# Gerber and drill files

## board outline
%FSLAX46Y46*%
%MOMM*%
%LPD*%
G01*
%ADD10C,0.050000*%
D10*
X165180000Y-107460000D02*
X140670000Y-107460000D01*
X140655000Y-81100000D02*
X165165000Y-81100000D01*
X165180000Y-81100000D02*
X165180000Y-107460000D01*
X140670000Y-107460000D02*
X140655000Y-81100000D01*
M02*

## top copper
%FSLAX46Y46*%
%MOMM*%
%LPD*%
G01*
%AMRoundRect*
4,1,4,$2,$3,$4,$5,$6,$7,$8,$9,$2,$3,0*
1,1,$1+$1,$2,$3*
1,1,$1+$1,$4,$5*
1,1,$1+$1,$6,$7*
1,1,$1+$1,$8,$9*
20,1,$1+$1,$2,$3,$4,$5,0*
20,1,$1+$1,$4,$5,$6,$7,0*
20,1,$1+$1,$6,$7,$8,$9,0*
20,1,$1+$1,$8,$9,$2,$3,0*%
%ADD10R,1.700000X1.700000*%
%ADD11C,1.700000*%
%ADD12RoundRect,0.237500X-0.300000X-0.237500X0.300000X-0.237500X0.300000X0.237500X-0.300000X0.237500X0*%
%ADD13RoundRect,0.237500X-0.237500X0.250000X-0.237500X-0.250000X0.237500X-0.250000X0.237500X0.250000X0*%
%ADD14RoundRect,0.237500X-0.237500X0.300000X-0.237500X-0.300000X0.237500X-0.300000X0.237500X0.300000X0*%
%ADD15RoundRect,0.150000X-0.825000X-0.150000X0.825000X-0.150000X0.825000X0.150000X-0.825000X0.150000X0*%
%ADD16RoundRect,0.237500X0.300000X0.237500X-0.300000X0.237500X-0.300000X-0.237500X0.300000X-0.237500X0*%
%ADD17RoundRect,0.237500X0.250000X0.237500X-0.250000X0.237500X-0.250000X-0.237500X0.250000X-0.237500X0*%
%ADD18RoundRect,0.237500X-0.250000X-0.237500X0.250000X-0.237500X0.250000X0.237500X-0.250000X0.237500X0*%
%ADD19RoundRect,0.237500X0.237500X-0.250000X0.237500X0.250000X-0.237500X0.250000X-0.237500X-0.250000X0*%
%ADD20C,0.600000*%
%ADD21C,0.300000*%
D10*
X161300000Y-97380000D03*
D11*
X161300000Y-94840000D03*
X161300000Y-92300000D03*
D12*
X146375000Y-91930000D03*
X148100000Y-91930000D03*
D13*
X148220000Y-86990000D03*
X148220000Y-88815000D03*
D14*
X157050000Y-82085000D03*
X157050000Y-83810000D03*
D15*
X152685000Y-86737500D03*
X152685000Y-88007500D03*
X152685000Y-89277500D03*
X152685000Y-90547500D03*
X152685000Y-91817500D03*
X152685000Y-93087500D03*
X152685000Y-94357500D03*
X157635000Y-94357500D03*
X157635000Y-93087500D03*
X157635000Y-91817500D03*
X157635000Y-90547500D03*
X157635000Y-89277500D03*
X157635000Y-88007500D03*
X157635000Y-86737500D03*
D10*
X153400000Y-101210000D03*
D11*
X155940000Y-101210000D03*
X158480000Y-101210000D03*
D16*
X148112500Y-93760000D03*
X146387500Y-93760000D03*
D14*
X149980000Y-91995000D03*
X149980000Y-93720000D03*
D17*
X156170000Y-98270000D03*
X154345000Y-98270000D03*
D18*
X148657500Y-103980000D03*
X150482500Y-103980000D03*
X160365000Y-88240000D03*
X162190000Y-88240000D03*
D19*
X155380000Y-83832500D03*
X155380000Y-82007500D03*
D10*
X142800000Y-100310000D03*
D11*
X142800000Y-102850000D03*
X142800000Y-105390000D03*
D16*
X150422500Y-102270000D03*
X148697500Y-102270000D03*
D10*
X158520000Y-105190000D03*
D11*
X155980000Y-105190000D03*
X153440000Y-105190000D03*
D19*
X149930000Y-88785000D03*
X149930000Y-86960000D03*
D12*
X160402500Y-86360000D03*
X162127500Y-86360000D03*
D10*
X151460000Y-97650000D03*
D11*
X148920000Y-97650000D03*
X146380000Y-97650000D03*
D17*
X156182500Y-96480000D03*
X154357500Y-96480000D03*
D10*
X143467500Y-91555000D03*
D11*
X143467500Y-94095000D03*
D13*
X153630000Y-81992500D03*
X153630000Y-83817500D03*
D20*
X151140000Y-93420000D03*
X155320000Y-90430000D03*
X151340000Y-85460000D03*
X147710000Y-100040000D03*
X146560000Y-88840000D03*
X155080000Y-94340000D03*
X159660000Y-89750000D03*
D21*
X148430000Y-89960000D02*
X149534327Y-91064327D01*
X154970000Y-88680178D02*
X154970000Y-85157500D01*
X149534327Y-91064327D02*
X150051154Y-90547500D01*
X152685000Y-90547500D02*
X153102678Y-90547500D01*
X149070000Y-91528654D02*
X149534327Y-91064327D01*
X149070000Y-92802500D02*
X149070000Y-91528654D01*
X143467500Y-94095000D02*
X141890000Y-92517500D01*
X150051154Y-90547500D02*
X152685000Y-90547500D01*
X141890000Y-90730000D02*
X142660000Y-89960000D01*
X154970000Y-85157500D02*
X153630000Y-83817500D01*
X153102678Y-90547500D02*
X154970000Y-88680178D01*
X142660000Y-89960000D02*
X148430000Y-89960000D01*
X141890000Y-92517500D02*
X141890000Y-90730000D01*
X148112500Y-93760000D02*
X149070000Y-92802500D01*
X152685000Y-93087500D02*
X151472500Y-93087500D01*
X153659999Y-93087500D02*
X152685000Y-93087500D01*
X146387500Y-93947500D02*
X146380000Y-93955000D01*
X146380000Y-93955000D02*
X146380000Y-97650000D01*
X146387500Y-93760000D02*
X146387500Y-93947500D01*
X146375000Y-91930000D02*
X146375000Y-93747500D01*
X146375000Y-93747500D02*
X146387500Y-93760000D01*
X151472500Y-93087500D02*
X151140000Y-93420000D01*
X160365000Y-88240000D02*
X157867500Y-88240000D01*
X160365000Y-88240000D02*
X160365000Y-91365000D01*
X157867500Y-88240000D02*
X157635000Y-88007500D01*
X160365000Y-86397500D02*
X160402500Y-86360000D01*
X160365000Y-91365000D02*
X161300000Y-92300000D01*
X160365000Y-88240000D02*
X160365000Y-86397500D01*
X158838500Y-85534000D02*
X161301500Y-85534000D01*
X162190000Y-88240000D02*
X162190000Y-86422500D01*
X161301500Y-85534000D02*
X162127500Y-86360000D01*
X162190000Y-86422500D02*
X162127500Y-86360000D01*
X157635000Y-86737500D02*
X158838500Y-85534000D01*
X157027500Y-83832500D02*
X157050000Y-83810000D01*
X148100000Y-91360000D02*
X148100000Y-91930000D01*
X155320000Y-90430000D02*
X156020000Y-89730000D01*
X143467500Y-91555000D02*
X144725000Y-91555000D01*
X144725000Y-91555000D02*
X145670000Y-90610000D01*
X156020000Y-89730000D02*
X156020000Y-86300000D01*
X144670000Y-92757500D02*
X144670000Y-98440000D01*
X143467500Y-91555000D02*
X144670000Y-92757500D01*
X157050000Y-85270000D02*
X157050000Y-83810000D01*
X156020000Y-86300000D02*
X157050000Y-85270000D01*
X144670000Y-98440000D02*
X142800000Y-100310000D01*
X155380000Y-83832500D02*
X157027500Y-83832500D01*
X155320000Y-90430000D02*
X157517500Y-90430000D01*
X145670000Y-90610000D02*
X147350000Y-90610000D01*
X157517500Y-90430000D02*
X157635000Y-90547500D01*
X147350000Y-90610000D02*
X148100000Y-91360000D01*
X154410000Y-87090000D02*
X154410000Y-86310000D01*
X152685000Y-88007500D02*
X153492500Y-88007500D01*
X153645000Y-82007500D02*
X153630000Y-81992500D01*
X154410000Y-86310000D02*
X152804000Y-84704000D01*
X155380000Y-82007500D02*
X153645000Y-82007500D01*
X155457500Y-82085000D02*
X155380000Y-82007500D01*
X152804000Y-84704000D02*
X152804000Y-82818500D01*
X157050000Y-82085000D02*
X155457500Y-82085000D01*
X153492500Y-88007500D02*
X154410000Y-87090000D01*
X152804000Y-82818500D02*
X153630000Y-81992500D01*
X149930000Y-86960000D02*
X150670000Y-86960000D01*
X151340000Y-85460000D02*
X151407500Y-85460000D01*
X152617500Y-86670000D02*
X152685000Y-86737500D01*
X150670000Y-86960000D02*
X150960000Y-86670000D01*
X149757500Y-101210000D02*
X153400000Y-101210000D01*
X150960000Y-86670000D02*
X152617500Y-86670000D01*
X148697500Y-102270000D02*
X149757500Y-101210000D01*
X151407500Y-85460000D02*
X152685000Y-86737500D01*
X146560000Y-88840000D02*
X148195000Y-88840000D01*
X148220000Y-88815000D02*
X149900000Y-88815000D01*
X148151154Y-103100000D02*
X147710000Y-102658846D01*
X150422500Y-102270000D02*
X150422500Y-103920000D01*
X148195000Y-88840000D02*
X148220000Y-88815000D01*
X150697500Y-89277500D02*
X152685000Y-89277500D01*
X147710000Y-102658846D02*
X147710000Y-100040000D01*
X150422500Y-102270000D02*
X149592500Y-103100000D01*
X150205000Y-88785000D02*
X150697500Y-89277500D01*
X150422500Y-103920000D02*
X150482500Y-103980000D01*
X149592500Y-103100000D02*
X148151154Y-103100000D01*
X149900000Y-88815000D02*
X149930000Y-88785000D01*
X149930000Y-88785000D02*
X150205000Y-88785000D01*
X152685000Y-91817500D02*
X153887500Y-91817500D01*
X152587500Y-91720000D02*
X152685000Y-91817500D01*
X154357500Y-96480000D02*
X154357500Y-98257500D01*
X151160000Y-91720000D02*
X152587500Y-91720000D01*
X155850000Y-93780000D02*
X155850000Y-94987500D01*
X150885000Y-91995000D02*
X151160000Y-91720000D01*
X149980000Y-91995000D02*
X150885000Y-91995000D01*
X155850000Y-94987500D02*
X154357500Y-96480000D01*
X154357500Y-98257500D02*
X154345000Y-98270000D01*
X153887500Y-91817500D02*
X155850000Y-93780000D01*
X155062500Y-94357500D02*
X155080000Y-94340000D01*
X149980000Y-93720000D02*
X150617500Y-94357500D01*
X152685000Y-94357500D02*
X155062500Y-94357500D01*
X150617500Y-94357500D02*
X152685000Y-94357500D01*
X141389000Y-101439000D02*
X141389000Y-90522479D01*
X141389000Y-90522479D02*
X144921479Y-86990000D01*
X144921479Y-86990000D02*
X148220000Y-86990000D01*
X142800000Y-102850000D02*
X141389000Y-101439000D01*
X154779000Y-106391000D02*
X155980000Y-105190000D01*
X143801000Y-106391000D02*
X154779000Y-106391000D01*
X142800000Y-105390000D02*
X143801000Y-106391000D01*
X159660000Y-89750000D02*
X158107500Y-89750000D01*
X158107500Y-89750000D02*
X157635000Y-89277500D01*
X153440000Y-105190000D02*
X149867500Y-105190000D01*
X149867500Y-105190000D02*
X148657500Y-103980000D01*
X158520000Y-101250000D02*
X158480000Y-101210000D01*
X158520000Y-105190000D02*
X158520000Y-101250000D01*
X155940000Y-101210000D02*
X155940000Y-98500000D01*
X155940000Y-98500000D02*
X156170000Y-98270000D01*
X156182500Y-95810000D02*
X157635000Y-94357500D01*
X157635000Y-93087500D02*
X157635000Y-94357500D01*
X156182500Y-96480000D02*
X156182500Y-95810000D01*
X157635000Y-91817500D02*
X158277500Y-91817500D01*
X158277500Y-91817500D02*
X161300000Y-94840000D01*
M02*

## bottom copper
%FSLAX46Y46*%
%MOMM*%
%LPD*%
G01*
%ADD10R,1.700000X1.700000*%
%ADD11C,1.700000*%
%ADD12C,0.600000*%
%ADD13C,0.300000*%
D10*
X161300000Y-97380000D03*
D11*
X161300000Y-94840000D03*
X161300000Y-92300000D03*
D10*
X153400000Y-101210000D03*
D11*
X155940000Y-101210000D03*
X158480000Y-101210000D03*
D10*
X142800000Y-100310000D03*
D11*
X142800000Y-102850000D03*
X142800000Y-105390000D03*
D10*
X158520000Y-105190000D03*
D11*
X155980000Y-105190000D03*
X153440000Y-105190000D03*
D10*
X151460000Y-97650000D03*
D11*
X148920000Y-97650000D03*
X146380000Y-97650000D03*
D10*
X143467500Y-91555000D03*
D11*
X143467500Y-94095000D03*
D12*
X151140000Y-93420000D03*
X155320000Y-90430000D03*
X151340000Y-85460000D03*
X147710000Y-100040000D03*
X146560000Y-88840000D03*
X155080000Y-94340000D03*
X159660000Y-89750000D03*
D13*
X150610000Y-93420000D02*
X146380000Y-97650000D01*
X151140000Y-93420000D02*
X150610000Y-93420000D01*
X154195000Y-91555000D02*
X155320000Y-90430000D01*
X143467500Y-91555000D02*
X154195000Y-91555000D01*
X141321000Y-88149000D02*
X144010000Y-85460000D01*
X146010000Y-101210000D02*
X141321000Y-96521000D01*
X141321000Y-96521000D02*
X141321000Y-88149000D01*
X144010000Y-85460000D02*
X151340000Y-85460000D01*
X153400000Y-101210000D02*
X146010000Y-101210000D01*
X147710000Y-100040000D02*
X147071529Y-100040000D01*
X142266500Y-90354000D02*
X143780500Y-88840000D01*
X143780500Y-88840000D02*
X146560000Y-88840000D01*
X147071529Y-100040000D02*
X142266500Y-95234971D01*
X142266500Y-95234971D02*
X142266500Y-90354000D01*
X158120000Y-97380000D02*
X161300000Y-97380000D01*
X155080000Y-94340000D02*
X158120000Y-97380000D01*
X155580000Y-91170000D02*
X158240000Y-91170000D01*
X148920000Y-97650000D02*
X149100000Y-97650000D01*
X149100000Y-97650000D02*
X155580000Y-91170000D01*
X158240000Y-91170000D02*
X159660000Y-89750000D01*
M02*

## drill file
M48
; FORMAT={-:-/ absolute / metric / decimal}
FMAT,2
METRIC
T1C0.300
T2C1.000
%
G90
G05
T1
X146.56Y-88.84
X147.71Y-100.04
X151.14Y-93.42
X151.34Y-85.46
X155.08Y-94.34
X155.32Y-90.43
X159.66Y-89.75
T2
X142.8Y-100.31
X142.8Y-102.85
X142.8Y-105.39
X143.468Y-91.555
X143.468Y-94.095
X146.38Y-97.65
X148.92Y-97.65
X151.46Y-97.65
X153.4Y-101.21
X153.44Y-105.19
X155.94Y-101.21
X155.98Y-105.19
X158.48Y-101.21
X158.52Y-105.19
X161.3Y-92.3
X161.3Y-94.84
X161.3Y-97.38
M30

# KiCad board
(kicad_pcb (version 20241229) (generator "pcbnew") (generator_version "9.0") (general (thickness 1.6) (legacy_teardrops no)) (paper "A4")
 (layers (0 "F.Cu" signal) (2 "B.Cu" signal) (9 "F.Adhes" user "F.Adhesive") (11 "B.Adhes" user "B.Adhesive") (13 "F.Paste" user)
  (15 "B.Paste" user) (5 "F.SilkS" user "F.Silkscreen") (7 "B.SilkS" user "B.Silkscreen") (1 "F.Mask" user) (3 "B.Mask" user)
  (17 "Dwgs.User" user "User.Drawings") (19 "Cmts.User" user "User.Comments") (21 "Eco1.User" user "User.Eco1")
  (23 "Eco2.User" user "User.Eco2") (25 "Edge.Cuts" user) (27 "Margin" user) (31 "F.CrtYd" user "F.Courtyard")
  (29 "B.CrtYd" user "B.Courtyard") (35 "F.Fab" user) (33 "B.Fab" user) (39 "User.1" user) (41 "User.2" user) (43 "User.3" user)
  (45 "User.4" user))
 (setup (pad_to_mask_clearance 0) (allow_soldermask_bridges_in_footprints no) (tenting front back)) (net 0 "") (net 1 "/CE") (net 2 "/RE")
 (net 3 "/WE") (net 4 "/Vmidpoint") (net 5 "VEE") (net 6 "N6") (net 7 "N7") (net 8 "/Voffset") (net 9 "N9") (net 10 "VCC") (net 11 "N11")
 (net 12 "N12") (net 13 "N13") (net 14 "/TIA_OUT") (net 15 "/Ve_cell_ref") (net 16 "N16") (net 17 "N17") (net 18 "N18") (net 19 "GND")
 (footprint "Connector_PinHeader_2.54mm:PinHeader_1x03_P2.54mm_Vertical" (layer "F.Cu") (at 161.3 97.38 180)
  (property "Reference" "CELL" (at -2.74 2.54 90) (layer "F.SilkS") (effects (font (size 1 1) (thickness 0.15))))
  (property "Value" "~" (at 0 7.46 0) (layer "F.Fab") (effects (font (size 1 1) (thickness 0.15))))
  (pad "1" thru_hole rect (at 0 0 180) (size 1.7 1.7) (drill 1) (layers "*.Cu" "*.Mask") (remove_unused_layers no) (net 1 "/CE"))
  (pad "2" thru_hole circle (at 0 2.54 180) (size 1.7 1.7) (drill 1) (layers "*.Cu" "*.Mask") (remove_unused_layers no) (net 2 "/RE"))
  (pad "3" thru_hole circle (at 0 5.08 180) (size 1.7 1.7) (drill 1) (layers "*.Cu" "*.Mask") (remove_unused_layers no) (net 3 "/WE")))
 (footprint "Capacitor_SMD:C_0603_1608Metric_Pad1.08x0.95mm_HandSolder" (layer "F.Cu") (at 147.2375 91.93)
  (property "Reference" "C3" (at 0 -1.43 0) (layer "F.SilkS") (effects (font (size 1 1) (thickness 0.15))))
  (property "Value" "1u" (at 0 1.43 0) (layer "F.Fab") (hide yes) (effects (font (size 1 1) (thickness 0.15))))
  (pad "1" smd roundrect (at -0.8625 0) (size 1.075 0.95) (layers "F.Cu" "F.Mask" "F.Paste") (roundrect_rratio 0.25) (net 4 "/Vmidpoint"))
  (pad "2" smd roundrect (at 0.8625 0) (size 1.075 0.95) (layers "F.Cu" "F.Mask" "F.Paste") (roundrect_rratio 0.25) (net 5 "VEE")))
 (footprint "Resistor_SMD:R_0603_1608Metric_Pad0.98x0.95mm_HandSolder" (layer "F.Cu") (at 148.22 87.9025 -90)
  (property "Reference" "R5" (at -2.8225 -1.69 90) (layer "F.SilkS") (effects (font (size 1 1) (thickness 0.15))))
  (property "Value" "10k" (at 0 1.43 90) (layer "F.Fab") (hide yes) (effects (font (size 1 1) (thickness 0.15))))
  (pad "1" smd roundrect (at -0.9125 0 270) (size 0.975 0.95) (layers "F.Cu" "F.Mask" "F.Paste") (roundrect_rratio 0.25) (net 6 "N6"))
  (pad "2" smd roundrect (at 0.9125 0 270) (size 0.975 0.95) (layers "F.Cu" "F.Mask" "F.Paste") (roundrect_rratio 0.25) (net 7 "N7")))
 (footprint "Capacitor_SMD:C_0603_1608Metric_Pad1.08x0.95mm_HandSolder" (layer "F.Cu") (at 157.05 82.9475 -90)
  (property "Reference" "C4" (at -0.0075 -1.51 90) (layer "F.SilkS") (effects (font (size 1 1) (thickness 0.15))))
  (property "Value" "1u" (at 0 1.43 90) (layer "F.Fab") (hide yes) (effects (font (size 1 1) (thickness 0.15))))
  (pad "1" smd roundrect (at -0.8625 0 270) (size 1.075 0.95) (layers "F.Cu" "F.Mask" "F.Paste") (roundrect_rratio 0.25) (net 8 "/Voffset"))
  (pad "2" smd roundrect (at 0.8625 0 270) (size 1.075 0.95) (layers "F.Cu" "F.Mask" "F.Paste") (roundrect_rratio 0.25) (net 5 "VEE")))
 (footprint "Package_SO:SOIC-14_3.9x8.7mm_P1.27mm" (layer "F.Cu") (at 155.16 90.5475)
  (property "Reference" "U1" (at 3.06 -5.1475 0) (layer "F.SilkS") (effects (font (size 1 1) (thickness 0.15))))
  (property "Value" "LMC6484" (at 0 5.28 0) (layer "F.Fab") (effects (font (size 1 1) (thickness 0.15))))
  (pad "1" smd roundrect (at -2.475 -3.81) (size 1.95 0.6) (layers "F.Cu" "F.Mask" "F.Paste") (roundrect_rratio 0.25) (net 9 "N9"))
  (pad "2" smd roundrect (at -2.475 -2.54) (size 1.95 0.6) (layers "F.Cu" "F.Mask" "F.Paste") (roundrect_rratio 0.25) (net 8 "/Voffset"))
  (pad "3" smd roundrect (at -2.475 -1.27) (size 1.95 0.6) (layers "F.Cu" "F.Mask" "F.Paste") (roundrect_rratio 0.25) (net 7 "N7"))
  (pad "4" smd roundrect (at -2.475 0) (size 1.95 0.6) (layers "F.Cu" "F.Mask" "F.Paste") (roundrect_rratio 0.25) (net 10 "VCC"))
  (pad "5" smd roundrect (at -2.475 1.27) (size 1.95 0.6) (layers "F.Cu" "F.Mask" "F.Paste") (roundrect_rratio 0.25) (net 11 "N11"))
  (pad "6" smd roundrect (at -2.475 2.54) (size 1.95 0.6) (layers "F.Cu" "F.Mask" "F.Paste") (roundrect_rratio 0.25) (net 4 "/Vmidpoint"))
  (pad "7" smd roundrect (at -2.475 3.81) (size 1.95 0.6) (layers "F.Cu" "F.Mask" "F.Paste") (roundrect_rratio 0.25) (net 1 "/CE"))
  (pad "8" smd roundrect (at 2.475 3.81) (size 1.95 0.6) (layers "F.Cu" "F.Mask" "F.Paste") (roundrect_rratio 0.25) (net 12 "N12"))
  (pad "9" smd roundrect (at 2.475 2.54) (size 1.95 0.6) (layers "F.Cu" "F.Mask" "F.Paste") (roundrect_rratio 0.25) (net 12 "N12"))
  (pad "10" smd roundrect (at 2.475 1.27) (size 1.95 0.6) (layers "F.Cu" "F.Mask" "F.Paste") (roundrect_rratio 0.25) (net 2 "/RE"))
  (pad "11" smd roundrect (at 2.475 0) (size 1.95 0.6) (layers "F.Cu" "F.Mask" "F.Paste") (roundrect_rratio 0.25) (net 5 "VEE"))
  (pad "12" smd roundrect (at 2.475 -1.27) (size 1.95 0.6) (layers "F.Cu" "F.Mask" "F.Paste") (roundrect_rratio 0.25) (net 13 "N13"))
  (pad "13" smd roundrect (at 2.475 -2.54) (size 1.95 0.6) (layers "F.Cu" "F.Mask" "F.Paste") (roundrect_rratio 0.25) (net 3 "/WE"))
  (pad "14" smd roundrect (at 2.475 -3.81) (size 1.95 0.6) (layers "F.Cu" "F.Mask" "F.Paste") (roundrect_rratio 0.25) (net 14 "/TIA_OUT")))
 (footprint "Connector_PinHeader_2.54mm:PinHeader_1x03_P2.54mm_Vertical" (layer "F.Cu") (at 153.4 101.21 90)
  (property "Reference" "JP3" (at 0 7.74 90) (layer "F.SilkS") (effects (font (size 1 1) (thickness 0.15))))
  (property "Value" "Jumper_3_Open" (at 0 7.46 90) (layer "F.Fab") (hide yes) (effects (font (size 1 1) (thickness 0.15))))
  (pad "1" thru_hole rect (at 0 0 90) (size 1.7 1.7) (drill 1) (layers "*.Cu" "*.Mask") (remove_unused_layers no) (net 9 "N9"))
  (pad "2" thru_hole circle (at 0 2.54 90) (size 1.7 1.7) (drill 1) (layers "*.Cu" "*.Mask") (remove_unused_layers no)
   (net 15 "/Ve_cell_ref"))
  (pad "3" thru_hole circle (at 0 5.08 90) (size 1.7 1.7) (drill 1) (layers "*.Cu" "*.Mask") (remove_unused_layers no) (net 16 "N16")))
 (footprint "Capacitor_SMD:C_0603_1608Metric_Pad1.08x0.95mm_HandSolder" (layer "F.Cu") (at 147.25 93.76 180)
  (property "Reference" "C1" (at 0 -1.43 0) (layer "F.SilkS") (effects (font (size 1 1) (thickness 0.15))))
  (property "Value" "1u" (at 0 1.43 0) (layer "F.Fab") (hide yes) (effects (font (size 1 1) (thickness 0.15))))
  (pad "1" smd roundrect (at -0.8625 0 180) (size 1.075 0.95) (layers "F.Cu" "F.Mask" "F.Paste") (roundrect_rratio 0.25) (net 10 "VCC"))
  (pad "2" smd roundrect (at 0.8625 0 180) (size 1.075 0.95) (layers "F.Cu" "F.Mask" "F.Paste") (roundrect_rratio 0.25) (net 4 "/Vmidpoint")))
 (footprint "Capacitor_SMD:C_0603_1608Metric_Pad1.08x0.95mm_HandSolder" (layer "F.Cu") (at 149.98 92.8575 -90)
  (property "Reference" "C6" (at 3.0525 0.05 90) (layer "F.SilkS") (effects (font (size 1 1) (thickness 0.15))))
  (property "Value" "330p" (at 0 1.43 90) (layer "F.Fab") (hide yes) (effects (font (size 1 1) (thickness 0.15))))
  (pad "1" smd roundrect (at -0.8625 0 270) (size 1.075 0.95) (layers "F.Cu" "F.Mask" "F.Paste") (roundrect_rratio 0.25) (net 11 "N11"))
  (pad "2" smd roundrect (at 0.8625 0 270) (size 1.075 0.95) (layers "F.Cu" "F.Mask" "F.Paste") (roundrect_rratio 0.25) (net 1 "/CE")))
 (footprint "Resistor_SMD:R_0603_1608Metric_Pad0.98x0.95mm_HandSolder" (layer "F.Cu") (at 155.2575 98.27 180)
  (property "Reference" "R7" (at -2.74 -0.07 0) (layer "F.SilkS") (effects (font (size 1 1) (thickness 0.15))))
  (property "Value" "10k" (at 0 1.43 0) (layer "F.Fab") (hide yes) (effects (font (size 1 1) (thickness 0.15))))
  (pad "1" smd roundrect (at -0.9125 0 180) (size 0.975 0.95) (layers "F.Cu" "F.Mask" "F.Paste") (roundrect_rratio 0.25)
   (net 15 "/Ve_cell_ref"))
  (pad "2" smd roundrect (at 0.9125 0 180) (size 0.975 0.95) (layers "F.Cu" "F.Mask" "F.Paste") (roundrect_rratio 0.25) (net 11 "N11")))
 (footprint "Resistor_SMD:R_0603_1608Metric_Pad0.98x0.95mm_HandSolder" (layer "F.Cu") (at 149.57 103.98)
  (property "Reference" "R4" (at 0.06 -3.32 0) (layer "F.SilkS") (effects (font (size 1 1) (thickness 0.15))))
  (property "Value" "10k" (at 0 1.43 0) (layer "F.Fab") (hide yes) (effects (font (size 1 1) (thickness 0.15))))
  (pad "1" smd roundrect (at -0.9125 0) (size 0.975 0.95) (layers "F.Cu" "F.Mask" "F.Paste") (roundrect_rratio 0.25) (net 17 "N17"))
  (pad "2" smd roundrect (at 0.9125 0) (size 0.975 0.95) (layers "F.Cu" "F.Mask" "F.Paste") (roundrect_rratio 0.25) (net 7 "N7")))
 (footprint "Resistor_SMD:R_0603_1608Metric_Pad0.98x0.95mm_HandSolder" (layer "F.Cu") (at 161.2775 88.24)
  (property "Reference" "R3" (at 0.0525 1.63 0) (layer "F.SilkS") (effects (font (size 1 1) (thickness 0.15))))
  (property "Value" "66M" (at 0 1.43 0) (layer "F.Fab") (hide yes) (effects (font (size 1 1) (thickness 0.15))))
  (pad "1" smd roundrect (at -0.9125 0) (size 0.975 0.95) (layers "F.Cu" "F.Mask" "F.Paste") (roundrect_rratio 0.25) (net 3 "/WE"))
  (pad "2" smd roundrect (at 0.9125 0) (size 0.975 0.95) (layers "F.Cu" "F.Mask" "F.Paste") (roundrect_rratio 0.25) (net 14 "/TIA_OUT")))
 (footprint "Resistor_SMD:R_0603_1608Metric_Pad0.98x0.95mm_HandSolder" (layer "F.Cu") (at 155.38 82.92 90)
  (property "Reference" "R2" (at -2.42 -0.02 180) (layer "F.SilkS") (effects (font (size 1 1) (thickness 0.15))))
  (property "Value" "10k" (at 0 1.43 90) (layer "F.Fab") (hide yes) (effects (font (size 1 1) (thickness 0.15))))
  (pad "1" smd roundrect (at -0.9125 0 90) (size 0.975 0.95) (layers "F.Cu" "F.Mask" "F.Paste") (roundrect_rratio 0.25) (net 5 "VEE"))
  (pad "2" smd roundrect (at 0.9125 0 90) (size 0.975 0.95) (layers "F.Cu" "F.Mask" "F.Paste") (roundrect_rratio 0.25) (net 8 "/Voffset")))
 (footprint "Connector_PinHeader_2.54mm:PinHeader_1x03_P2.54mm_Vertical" (layer "F.Cu") (at 142.8 100.31)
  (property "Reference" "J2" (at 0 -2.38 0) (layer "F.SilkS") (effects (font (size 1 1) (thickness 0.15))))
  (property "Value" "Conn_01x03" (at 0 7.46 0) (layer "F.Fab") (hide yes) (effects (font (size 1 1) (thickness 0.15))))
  (pad "1" thru_hole rect (at 0 0) (size 1.7 1.7) (drill 1) (layers "*.Cu" "*.Mask") (remove_unused_layers no) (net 5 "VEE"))
  (pad "2" thru_hole circle (at 0 2.54) (size 1.7 1.7) (drill 1) (layers "*.Cu" "*.Mask") (remove_unused_layers no) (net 6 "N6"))
  (pad "3" thru_hole circle (at 0 5.08) (size 1.7 1.7) (drill 1) (layers "*.Cu" "*.Mask") (remove_unused_layers no) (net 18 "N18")))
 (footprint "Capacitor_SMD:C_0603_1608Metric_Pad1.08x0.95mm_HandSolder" (layer "F.Cu") (at 149.56 102.27 180)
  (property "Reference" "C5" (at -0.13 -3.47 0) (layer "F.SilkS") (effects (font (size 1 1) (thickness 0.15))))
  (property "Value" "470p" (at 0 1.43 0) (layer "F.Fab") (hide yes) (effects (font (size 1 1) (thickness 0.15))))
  (pad "1" smd roundrect (at -0.8625 0 180) (size 1.075 0.95) (layers "F.Cu" "F.Mask" "F.Paste") (roundrect_rratio 0.25) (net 7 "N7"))
  (pad "2" smd roundrect (at 0.8625 0 180) (size 1.075 0.95) (layers "F.Cu" "F.Mask" "F.Paste") (roundrect_rratio 0.25) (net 9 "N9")))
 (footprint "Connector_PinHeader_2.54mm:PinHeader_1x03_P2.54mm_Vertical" (layer "F.Cu") (at 158.52 105.19 -90)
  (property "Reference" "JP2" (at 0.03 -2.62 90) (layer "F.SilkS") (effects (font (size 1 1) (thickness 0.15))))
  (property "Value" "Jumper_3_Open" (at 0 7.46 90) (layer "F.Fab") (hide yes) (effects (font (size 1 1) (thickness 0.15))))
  (pad "1" thru_hole rect (at 0 0 270) (size 1.7 1.7) (drill 1) (layers "*.Cu" "*.Mask") (remove_unused_layers no) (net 16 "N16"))
  (pad "2" thru_hole circle (at 0 2.54 270) (size 1.7 1.7) (drill 1) (layers "*.Cu" "*.Mask") (remove_unused_layers no) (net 18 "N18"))
  (pad "3" thru_hole circle (at 0 5.08 270) (size 1.7 1.7) (drill 1) (layers "*.Cu" "*.Mask") (remove_unused_layers no) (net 17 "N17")))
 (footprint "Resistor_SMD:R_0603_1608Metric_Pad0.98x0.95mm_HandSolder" (layer "F.Cu") (at 149.93 87.8725 90)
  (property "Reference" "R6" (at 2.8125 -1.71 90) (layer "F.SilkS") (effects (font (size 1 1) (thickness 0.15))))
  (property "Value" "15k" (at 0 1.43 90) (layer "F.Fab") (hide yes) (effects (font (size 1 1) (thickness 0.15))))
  (pad "1" smd roundrect (at -0.9125 0 90) (size 0.975 0.95) (layers "F.Cu" "F.Mask" "F.Paste") (roundrect_rratio 0.25) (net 7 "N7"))
  (pad "2" smd roundrect (at 0.9125 0 90) (size 0.975 0.95) (layers "F.Cu" "F.Mask" "F.Paste") (roundrect_rratio 0.25) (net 9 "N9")))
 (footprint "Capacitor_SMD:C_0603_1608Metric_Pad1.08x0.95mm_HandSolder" (layer "F.Cu") (at 161.265 86.36)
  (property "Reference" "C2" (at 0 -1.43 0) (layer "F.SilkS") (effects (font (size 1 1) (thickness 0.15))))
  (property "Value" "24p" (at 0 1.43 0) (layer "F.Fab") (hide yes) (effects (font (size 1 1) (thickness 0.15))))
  (pad "1" smd roundrect (at -0.8625 0) (size 1.075 0.95) (layers "F.Cu" "F.Mask" "F.Paste") (roundrect_rratio 0.25) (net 3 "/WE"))
  (pad "2" smd roundrect (at 0.8625 0) (size 1.075 0.95) (layers "F.Cu" "F.Mask" "F.Paste") (roundrect_rratio 0.25) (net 14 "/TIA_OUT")))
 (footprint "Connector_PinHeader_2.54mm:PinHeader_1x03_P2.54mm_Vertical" (layer "F.Cu") (at 151.46 97.65 -90)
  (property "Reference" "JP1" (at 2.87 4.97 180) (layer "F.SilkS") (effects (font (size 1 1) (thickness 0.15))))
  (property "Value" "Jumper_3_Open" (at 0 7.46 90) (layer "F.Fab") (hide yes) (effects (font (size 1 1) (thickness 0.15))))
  (pad "1" thru_hole rect (at 0 0 270) (size 1.7 1.7) (drill 1) (layers "*.Cu" "*.Mask") (remove_unused_layers no) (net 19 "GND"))
  (pad "2" thru_hole circle (at 0 2.54 270) (size 1.7 1.7) (drill 1) (layers "*.Cu" "*.Mask") (remove_unused_layers no) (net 13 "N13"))
  (pad "3" thru_hole circle (at 0 5.08 270) (size 1.7 1.7) (drill 1) (layers "*.Cu" "*.Mask") (remove_unused_layers no) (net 4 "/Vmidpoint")))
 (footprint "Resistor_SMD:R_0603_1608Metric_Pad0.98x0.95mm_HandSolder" (layer "F.Cu") (at 155.27 96.48 180)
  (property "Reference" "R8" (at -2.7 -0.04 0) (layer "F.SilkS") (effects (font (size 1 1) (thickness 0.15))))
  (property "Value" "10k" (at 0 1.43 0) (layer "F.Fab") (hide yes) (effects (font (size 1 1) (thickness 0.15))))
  (pad "1" smd roundrect (at -0.9125 0 180) (size 0.975 0.95) (layers "F.Cu" "F.Mask" "F.Paste") (roundrect_rratio 0.25) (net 12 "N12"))
  (pad "2" smd roundrect (at 0.9125 0 180) (size 0.975 0.95) (layers "F.Cu" "F.Mask" "F.Paste") (roundrect_rratio 0.25) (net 11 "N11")))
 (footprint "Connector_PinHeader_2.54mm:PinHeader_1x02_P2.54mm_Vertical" (layer "F.Cu") (at 143.4675 91.555)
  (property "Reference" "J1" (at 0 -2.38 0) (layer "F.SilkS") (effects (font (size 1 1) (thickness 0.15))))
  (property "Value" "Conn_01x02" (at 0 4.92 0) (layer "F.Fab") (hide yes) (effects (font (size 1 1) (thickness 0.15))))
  (pad "1" thru_hole rect (at 0 0) (size 1.7 1.7) (drill 1) (layers "*.Cu" "*.Mask") (remove_unused_layers no) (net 5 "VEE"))
  (pad "2" thru_hole circle (at 0 2.54) (size 1.7 1.7) (drill 1) (layers "*.Cu" "*.Mask") (remove_unused_layers no) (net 10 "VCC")))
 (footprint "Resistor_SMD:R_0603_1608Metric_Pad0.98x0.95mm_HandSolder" (layer "F.Cu") (at 153.63 82.905 -90)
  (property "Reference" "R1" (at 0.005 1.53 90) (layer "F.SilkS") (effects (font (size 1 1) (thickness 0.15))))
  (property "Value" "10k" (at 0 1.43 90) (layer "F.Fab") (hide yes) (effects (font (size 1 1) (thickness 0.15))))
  (pad "1" smd roundrect (at -0.9125 0 270) (size 0.975 0.95) (layers "F.Cu" "F.Mask" "F.Paste") (roundrect_rratio 0.25) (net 8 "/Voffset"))
  (pad "2" smd roundrect (at 0.9125 0 270) (size 0.975 0.95) (layers "F.Cu" "F.Mask" "F.Paste") (roundrect_rratio 0.25) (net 10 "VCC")))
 (gr_line (start 165.18 107.46) (end 140.67 107.46) (stroke (width 0.05) (type default)) (layer "Edge.Cuts"))
 (gr_line (start 140.655 81.1) (end 165.165 81.1) (stroke (width 0.05) (type default)) (layer "Edge.Cuts"))
 (gr_line (start 165.18 81.1) (end 165.18 107.46) (stroke (width 0.05) (type default)) (layer "Edge.Cuts"))
 (gr_line (start 140.67 107.46) (end 140.655 81.1) (stroke (width 0.05) (type default)) (layer "Edge.Cuts"))
 (segment (start 148.43 89.96) (end 149.534327 91.064327) (width 0.3) (layer "F.Cu") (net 10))
 (segment (start 154.97 88.680178) (end 154.97 85.1575) (width 0.3) (layer "F.Cu") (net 10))
 (segment (start 149.534327 91.064327) (end 150.051154 90.5475) (width 0.3) (layer "F.Cu") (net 10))
 (segment (start 152.685 90.5475) (end 153.102678 90.5475) (width 0.3) (layer "F.Cu") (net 10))
 (segment (start 149.07 91.528654) (end 149.534327 91.064327) (width 0.3) (layer "F.Cu") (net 10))
 (segment (start 149.07 92.8025) (end 149.07 91.528654) (width 0.3) (layer "F.Cu") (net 10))
 (segment (start 143.4675 94.095) (end 141.89 92.5175) (width 0.3) (layer "F.Cu") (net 10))
 (segment (start 150.051154 90.5475) (end 152.685 90.5475) (width 0.3) (layer "F.Cu") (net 10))
 (segment (start 141.89 90.73) (end 142.66 89.96) (width 0.3) (layer "F.Cu") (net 10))
 (segment (start 154.97 85.1575) (end 153.63 83.8175) (width 0.3) (layer "F.Cu") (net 10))
 (segment (start 153.102678 90.5475) (end 154.97 88.680178) (width 0.3) (layer "F.Cu") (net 10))
 (segment (start 142.66 89.96) (end 148.43 89.96) (width 0.3) (layer "F.Cu") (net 10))
 (segment (start 141.89 92.5175) (end 141.89 90.73) (width 0.3) (layer "F.Cu") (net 10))
 (segment (start 148.1125 93.76) (end 149.07 92.8025) (width 0.3) (layer "F.Cu") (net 10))
 (segment (start 152.685 93.0875) (end 151.4725 93.0875) (width 0.3) (layer "F.Cu") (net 4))
 (segment (start 153.659999 93.0875) (end 152.685 93.0875) (width 0.3) (layer "F.Cu") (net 4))
 (segment (start 146.3875 93.9475) (end 146.38 93.955) (width 0.3) (layer "F.Cu") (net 4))
 (segment (start 146.38 93.955) (end 146.38 97.65) (width 0.3) (layer "F.Cu") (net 4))
 (segment (start 146.3875 93.76) (end 146.3875 93.9475) (width 0.3) (layer "F.Cu") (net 4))
 (segment (start 146.375 91.93) (end 146.375 93.7475) (width 0.3) (layer "F.Cu") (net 4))
 (segment (start 146.375 93.7475) (end 146.3875 93.76) (width 0.3) (layer "F.Cu") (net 4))
 (segment (start 151.4725 93.0875) (end 151.14 93.42) (width 0.3) (layer "F.Cu") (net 4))
 (via (at 151.14 93.42) (size 0.6) (drill 0.3) (layers "F.Cu" "B.Cu") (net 4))
 (segment (start 150.61 93.42) (end 146.38 97.65) (width 0.3) (layer "B.Cu") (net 4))
 (segment (start 151.14 93.42) (end 150.61 93.42) (width 0.3) (layer "B.Cu") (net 4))
 (segment (start 160.365 88.24) (end 157.8675 88.24) (width 0.3) (layer "F.Cu") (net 3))
 (segment (start 160.365 88.24) (end 160.365 91.365) (width 0.3) (layer "F.Cu") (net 3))
 (segment (start 157.8675 88.24) (end 157.635 88.0075) (width 0.3) (layer "F.Cu") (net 3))
 (segment (start 160.365 86.3975) (end 160.4025 86.36) (width 0.3) (layer "F.Cu") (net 3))
 (segment (start 160.365 91.365) (end 161.3 92.3) (width 0.3) (layer "F.Cu") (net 3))
 (segment (start 160.365 88.24) (end 160.365 86.3975) (width 0.3) (layer "F.Cu") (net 3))
 (segment (start 158.8385 85.534) (end 161.3015 85.534) (width 0.3) (layer "F.Cu") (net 14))
 (segment (start 162.19 88.24) (end 162.19 86.4225) (width 0.3) (layer "F.Cu") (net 14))
 (segment (start 161.3015 85.534) (end 162.1275 86.36) (width 0.3) (layer "F.Cu") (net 14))
 (segment (start 162.19 86.4225) (end 162.1275 86.36) (width 0.3) (layer "F.Cu") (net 14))
 (segment (start 157.635 86.7375) (end 158.8385 85.534) (width 0.3) (layer "F.Cu") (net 14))
 (segment (start 157.0275 83.8325) (end 157.05 83.81) (width 0.3) (layer "F.Cu") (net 5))
 (segment (start 148.1 91.36) (end 148.1 91.93) (width 0.3) (layer "F.Cu") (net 5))
 (segment (start 155.32 90.43) (end 156.02 89.73) (width 0.3) (layer "F.Cu") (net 5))
 (segment (start 143.4675 91.555) (end 144.725 91.555) (width 0.3) (layer "F.Cu") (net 5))
 (segment (start 144.725 91.555) (end 145.67 90.61) (width 0.3) (layer "F.Cu") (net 5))
 (segment (start 156.02 89.73) (end 156.02 86.3) (width 0.3) (layer "F.Cu") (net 5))
 (segment (start 144.67 92.7575) (end 144.67 98.44) (width 0.3) (layer "F.Cu") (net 5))
 (segment (start 143.4675 91.555) (end 144.67 92.7575) (width 0.3) (layer "F.Cu") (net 5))
 (segment (start 157.05 85.27) (end 157.05 83.81) (width 0.3) (layer "F.Cu") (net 5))
 (segment (start 156.02 86.3) (end 157.05 85.27) (width 0.3) (layer "F.Cu") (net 5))
 (segment (start 144.67 98.44) (end 142.8 100.31) (width 0.3) (layer "F.Cu") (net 5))
 (segment (start 155.38 83.8325) (end 157.0275 83.8325) (width 0.3) (layer "F.Cu") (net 5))
 (segment (start 155.32 90.43) (end 157.5175 90.43) (width 0.3) (layer "F.Cu") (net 5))
 (segment (start 145.67 90.61) (end 147.35 90.61) (width 0.3) (layer "F.Cu") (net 5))
 (segment (start 157.5175 90.43) (end 157.635 90.5475) (width 0.3) (layer "F.Cu") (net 5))
 (segment (start 147.35 90.61) (end 148.1 91.36) (width 0.3) (layer "F.Cu") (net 5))
 (via (at 155.32 90.43) (size 0.6) (drill 0.3) (layers "F.Cu" "B.Cu") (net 5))
 (segment (start 154.195 91.555) (end 155.32 90.43) (width 0.3) (layer "B.Cu") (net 5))
 (segment (start 143.4675 91.555) (end 154.195 91.555) (width 0.3) (layer "B.Cu") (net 5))
 (segment (start 154.41 87.09) (end 154.41 86.31) (width 0.3) (layer "F.Cu") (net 8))
 (segment (start 152.685 88.0075) (end 153.4925 88.0075) (width 0.3) (layer "F.Cu") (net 8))
 (segment (start 153.645 82.0075) (end 153.63 81.9925) (width 0.3) (layer "F.Cu") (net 8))
 (segment (start 154.41 86.31) (end 152.804 84.704) (width 0.3) (layer "F.Cu") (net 8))
 (segment (start 155.38 82.0075) (end 153.645 82.0075) (width 0.3) (layer "F.Cu") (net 8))
 (segment (start 155.4575 82.085) (end 155.38 82.0075) (width 0.3) (layer "F.Cu") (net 8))
 (segment (start 152.804 84.704) (end 152.804 82.8185) (width 0.3) (layer "F.Cu") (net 8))
 (segment (start 157.05 82.085) (end 155.4575 82.085) (width 0.3) (layer "F.Cu") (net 8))
 (segment (start 153.4925 88.0075) (end 154.41 87.09) (width 0.3) (layer "F.Cu") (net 8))
 (segment (start 152.804 82.8185) (end 153.63 81.9925) (width 0.3) (layer "F.Cu") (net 8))
 (segment (start 149.93 86.96) (end 150.67 86.96) (width 0.3) (layer "F.Cu") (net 9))
 (segment (start 151.34 85.46) (end 151.4075 85.46) (width 0.3) (layer "F.Cu") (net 9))
 (segment (start 152.6175 86.67) (end 152.685 86.7375) (width 0.3) (layer "F.Cu") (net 9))
 (segment (start 150.67 86.96) (end 150.96 86.67) (width 0.3) (layer "F.Cu") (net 9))
 (segment (start 149.7575 101.21) (end 153.4 101.21) (width 0.3) (layer "F.Cu") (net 9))
 (segment (start 150.96 86.67) (end 152.6175 86.67) (width 0.3) (layer "F.Cu") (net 9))
 (segment (start 148.6975 102.27) (end 149.7575 101.21) (width 0.3) (layer "F.Cu") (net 9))
 (segment (start 151.4075 85.46) (end 152.685 86.7375) (width 0.3) (layer "F.Cu") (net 9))
 (via (at 151.34 85.46) (size 0.6) (drill 0.3) (layers "F.Cu" "B.Cu") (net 9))
 (segment (start 141.321 88.149) (end 144.01 85.46) (width 0.3) (layer "B.Cu") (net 9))
 (segment (start 146.01 101.21) (end 141.321 96.521) (width 0.3) (layer "B.Cu") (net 9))
 (segment (start 141.321 96.521) (end 141.321 88.149) (width 0.3) (layer "B.Cu") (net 9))
 (segment (start 144.01 85.46) (end 151.34 85.46) (width 0.3) (layer "B.Cu") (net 9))
 (segment (start 153.4 101.21) (end 146.01 101.21) (width 0.3) (layer "B.Cu") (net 9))
 (segment (start 146.56 88.84) (end 148.195 88.84) (width 0.3) (layer "F.Cu") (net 7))
 (segment (start 148.22 88.815) (end 149.9 88.815) (width 0.3) (layer "F.Cu") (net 7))
 (segment (start 148.151154 103.1) (end 147.71 102.658846) (width 0.3) (layer "F.Cu") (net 7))
 (segment (start 150.4225 102.27) (end 150.4225 103.92) (width 0.3) (layer "F.Cu") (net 7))
 (segment (start 148.195 88.84) (end 148.22 88.815) (width 0.3) (layer "F.Cu") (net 7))
 (segment (start 150.6975 89.2775) (end 152.685 89.2775) (width 0.3) (layer "F.Cu") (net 7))
 (segment (start 147.71 102.658846) (end 147.71 100.04) (width 0.3) (layer "F.Cu") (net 7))
 (segment (start 150.4225 102.27) (end 149.5925 103.1) (width 0.3) (layer "F.Cu") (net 7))
 (segment (start 150.205 88.785) (end 150.6975 89.2775) (width 0.3) (layer "F.Cu") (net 7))
 (segment (start 150.4225 103.92) (end 150.4825 103.98) (width 0.3) (layer "F.Cu") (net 7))
 (segment (start 149.5925 103.1) (end 148.151154 103.1) (width 0.3) (layer "F.Cu") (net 7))
 (segment (start 149.9 88.815) (end 149.93 88.785) (width 0.3) (layer "F.Cu") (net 7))
 (segment (start 149.93 88.785) (end 150.205 88.785) (width 0.3) (layer "F.Cu") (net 7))
 (via (at 147.71 100.04) (size 0.6) (drill 0.3) (layers "F.Cu" "B.Cu") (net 7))
 (via (at 146.56 88.84) (size 0.6) (drill 0.3) (layers "F.Cu" "B.Cu") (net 7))
 (segment (start 147.71 100.04) (end 147.071529 100.04) (width 0.3) (layer "B.Cu") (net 7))
 (segment (start 142.2665 90.354) (end 143.7805 88.84) (width 0.3) (layer "B.Cu") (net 7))
 (segment (start 143.7805 88.84) (end 146.56 88.84) (width 0.3) (layer "B.Cu") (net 7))
 (segment (start 147.071529 100.04) (end 142.2665 95.234971) (width 0.3) (layer "B.Cu") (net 7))
 (segment (start 142.2665 95.234971) (end 142.2665 90.354) (width 0.3) (layer "B.Cu") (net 7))
 (segment (start 152.685 91.8175) (end 153.8875 91.8175) (width 0.3) (layer "F.Cu") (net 11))
 (segment (start 152.5875 91.72) (end 152.685 91.8175) (width 0.3) (layer "F.Cu") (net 11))
 (segment (start 154.3575 96.48) (end 154.3575 98.2575) (width 0.3) (layer "F.Cu") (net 11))
 (segment (start 151.16 91.72) (end 152.5875 91.72) (width 0.3) (layer "F.Cu") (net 11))
 (segment (start 155.85 93.78) (end 155.85 94.9875) (width 0.3) (layer "F.Cu") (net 11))
 (segment (start 150.885 91.995) (end 151.16 91.72) (width 0.3) (layer "F.Cu") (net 11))
 (segment (start 149.98 91.995) (end 150.885 91.995) (width 0.3) (layer "F.Cu") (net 11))
 (segment (start 155.85 94.9875) (end 154.3575 96.48) (width 0.3) (layer "F.Cu") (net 11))
 (segment (start 154.3575 98.2575) (end 154.345 98.27) (width 0.3) (layer "F.Cu") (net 11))
 (segment (start 153.8875 91.8175) (end 155.85 93.78) (width 0.3) (layer "F.Cu") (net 11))
 (segment (start 155.0625 94.3575) (end 155.08 94.34) (width 0.3) (layer "F.Cu") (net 1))
 (segment (start 149.98 93.72) (end 150.6175 94.3575) (width 0.3) (layer "F.Cu") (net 1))
 (segment (start 152.685 94.3575) (end 155.0625 94.3575) (width 0.3) (layer "F.Cu") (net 1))
 (segment (start 150.6175 94.3575) (end 152.685 94.3575) (width 0.3) (layer "F.Cu") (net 1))
 (via (at 155.08 94.34) (size 0.6) (drill 0.3) (layers "F.Cu" "B.Cu") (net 1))
 (segment (start 158.12 97.38) (end 161.3 97.38) (width 0.3) (layer "B.Cu") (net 1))
 (segment (start 155.08 94.34) (end 158.12 97.38) (width 0.3) (layer "B.Cu") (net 1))
 (segment (start 141.389 101.439) (end 141.389 90.522479) (width 0.3) (layer "F.Cu") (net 6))
 (segment (start 141.389 90.522479) (end 144.921479 86.99) (width 0.3) (layer "F.Cu") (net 6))
 (segment (start 144.921479 86.99) (end 148.22 86.99) (width 0.3) (layer "F.Cu") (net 6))
 (segment (start 142.8 102.85) (end 141.389 101.439) (width 0.3) (layer "F.Cu") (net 6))
 (segment (start 154.779 106.391) (end 155.98 105.19) (width 0.3) (layer "F.Cu") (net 18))
 (segment (start 143.801 106.391) (end 154.779 106.391) (width 0.3) (layer "F.Cu") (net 18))
 (segment (start 142.8 105.39) (end 143.801 106.391) (width 0.3) (layer "F.Cu") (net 18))
 (segment (start 159.66 89.75) (end 158.1075 89.75) (width 0.3) (layer "F.Cu") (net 13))
 (segment (start 158.1075 89.75) (end 157.635 89.2775) (width 0.3) (layer "F.Cu") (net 13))
 (via (at 159.66 89.75) (size 0.6) (drill 0.3) (layers "F.Cu" "B.Cu") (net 13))
 (segment (start 155.58 91.17) (end 158.24 91.17) (width 0.3) (layer "B.Cu") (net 13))
 (segment (start 148.92 97.65) (end 149.1 97.65) (width 0.3) (layer "B.Cu") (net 13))
 (segment (start 149.1 97.65) (end 155.58 91.17) (width 0.3) (layer "B.Cu") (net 13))
 (segment (start 158.24 91.17) (end 159.66 89.75) (width 0.3) (layer "B.Cu") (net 13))
 (segment (start 153.44 105.19) (end 149.8675 105.19) (width 0.3) (layer "F.Cu") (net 17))
 (segment (start 149.8675 105.19) (end 148.6575 103.98) (width 0.3) (layer "F.Cu") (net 17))
 (segment (start 158.52 101.25) (end 158.48 101.21) (width 0.3) (layer "F.Cu") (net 16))
 (segment (start 158.52 105.19) (end 158.52 101.25) (width 0.3) (layer "F.Cu") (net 16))
 (segment (start 155.94 101.21) (end 155.94 98.5) (width 0.3) (layer "F.Cu") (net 15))
 (segment (start 155.94 98.5) (end 156.17 98.27) (width 0.3) (layer "F.Cu") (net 15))
 (segment (start 156.1825 95.81) (end 157.635 94.3575) (width 0.3) (layer "F.Cu") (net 12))
 (segment (start 157.635 93.0875) (end 157.635 94.3575) (width 0.3) (layer "F.Cu") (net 12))
 (segment (start 156.1825 96.48) (end 156.1825 95.81) (width 0.3) (layer "F.Cu") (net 12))
 (segment (start 157.635 91.8175) (end 158.2775 91.8175) (width 0.3) (layer "F.Cu") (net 2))
 (segment (start 158.2775 91.8175) (end 161.3 94.84) (width 0.3) (layer "F.Cu") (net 2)))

